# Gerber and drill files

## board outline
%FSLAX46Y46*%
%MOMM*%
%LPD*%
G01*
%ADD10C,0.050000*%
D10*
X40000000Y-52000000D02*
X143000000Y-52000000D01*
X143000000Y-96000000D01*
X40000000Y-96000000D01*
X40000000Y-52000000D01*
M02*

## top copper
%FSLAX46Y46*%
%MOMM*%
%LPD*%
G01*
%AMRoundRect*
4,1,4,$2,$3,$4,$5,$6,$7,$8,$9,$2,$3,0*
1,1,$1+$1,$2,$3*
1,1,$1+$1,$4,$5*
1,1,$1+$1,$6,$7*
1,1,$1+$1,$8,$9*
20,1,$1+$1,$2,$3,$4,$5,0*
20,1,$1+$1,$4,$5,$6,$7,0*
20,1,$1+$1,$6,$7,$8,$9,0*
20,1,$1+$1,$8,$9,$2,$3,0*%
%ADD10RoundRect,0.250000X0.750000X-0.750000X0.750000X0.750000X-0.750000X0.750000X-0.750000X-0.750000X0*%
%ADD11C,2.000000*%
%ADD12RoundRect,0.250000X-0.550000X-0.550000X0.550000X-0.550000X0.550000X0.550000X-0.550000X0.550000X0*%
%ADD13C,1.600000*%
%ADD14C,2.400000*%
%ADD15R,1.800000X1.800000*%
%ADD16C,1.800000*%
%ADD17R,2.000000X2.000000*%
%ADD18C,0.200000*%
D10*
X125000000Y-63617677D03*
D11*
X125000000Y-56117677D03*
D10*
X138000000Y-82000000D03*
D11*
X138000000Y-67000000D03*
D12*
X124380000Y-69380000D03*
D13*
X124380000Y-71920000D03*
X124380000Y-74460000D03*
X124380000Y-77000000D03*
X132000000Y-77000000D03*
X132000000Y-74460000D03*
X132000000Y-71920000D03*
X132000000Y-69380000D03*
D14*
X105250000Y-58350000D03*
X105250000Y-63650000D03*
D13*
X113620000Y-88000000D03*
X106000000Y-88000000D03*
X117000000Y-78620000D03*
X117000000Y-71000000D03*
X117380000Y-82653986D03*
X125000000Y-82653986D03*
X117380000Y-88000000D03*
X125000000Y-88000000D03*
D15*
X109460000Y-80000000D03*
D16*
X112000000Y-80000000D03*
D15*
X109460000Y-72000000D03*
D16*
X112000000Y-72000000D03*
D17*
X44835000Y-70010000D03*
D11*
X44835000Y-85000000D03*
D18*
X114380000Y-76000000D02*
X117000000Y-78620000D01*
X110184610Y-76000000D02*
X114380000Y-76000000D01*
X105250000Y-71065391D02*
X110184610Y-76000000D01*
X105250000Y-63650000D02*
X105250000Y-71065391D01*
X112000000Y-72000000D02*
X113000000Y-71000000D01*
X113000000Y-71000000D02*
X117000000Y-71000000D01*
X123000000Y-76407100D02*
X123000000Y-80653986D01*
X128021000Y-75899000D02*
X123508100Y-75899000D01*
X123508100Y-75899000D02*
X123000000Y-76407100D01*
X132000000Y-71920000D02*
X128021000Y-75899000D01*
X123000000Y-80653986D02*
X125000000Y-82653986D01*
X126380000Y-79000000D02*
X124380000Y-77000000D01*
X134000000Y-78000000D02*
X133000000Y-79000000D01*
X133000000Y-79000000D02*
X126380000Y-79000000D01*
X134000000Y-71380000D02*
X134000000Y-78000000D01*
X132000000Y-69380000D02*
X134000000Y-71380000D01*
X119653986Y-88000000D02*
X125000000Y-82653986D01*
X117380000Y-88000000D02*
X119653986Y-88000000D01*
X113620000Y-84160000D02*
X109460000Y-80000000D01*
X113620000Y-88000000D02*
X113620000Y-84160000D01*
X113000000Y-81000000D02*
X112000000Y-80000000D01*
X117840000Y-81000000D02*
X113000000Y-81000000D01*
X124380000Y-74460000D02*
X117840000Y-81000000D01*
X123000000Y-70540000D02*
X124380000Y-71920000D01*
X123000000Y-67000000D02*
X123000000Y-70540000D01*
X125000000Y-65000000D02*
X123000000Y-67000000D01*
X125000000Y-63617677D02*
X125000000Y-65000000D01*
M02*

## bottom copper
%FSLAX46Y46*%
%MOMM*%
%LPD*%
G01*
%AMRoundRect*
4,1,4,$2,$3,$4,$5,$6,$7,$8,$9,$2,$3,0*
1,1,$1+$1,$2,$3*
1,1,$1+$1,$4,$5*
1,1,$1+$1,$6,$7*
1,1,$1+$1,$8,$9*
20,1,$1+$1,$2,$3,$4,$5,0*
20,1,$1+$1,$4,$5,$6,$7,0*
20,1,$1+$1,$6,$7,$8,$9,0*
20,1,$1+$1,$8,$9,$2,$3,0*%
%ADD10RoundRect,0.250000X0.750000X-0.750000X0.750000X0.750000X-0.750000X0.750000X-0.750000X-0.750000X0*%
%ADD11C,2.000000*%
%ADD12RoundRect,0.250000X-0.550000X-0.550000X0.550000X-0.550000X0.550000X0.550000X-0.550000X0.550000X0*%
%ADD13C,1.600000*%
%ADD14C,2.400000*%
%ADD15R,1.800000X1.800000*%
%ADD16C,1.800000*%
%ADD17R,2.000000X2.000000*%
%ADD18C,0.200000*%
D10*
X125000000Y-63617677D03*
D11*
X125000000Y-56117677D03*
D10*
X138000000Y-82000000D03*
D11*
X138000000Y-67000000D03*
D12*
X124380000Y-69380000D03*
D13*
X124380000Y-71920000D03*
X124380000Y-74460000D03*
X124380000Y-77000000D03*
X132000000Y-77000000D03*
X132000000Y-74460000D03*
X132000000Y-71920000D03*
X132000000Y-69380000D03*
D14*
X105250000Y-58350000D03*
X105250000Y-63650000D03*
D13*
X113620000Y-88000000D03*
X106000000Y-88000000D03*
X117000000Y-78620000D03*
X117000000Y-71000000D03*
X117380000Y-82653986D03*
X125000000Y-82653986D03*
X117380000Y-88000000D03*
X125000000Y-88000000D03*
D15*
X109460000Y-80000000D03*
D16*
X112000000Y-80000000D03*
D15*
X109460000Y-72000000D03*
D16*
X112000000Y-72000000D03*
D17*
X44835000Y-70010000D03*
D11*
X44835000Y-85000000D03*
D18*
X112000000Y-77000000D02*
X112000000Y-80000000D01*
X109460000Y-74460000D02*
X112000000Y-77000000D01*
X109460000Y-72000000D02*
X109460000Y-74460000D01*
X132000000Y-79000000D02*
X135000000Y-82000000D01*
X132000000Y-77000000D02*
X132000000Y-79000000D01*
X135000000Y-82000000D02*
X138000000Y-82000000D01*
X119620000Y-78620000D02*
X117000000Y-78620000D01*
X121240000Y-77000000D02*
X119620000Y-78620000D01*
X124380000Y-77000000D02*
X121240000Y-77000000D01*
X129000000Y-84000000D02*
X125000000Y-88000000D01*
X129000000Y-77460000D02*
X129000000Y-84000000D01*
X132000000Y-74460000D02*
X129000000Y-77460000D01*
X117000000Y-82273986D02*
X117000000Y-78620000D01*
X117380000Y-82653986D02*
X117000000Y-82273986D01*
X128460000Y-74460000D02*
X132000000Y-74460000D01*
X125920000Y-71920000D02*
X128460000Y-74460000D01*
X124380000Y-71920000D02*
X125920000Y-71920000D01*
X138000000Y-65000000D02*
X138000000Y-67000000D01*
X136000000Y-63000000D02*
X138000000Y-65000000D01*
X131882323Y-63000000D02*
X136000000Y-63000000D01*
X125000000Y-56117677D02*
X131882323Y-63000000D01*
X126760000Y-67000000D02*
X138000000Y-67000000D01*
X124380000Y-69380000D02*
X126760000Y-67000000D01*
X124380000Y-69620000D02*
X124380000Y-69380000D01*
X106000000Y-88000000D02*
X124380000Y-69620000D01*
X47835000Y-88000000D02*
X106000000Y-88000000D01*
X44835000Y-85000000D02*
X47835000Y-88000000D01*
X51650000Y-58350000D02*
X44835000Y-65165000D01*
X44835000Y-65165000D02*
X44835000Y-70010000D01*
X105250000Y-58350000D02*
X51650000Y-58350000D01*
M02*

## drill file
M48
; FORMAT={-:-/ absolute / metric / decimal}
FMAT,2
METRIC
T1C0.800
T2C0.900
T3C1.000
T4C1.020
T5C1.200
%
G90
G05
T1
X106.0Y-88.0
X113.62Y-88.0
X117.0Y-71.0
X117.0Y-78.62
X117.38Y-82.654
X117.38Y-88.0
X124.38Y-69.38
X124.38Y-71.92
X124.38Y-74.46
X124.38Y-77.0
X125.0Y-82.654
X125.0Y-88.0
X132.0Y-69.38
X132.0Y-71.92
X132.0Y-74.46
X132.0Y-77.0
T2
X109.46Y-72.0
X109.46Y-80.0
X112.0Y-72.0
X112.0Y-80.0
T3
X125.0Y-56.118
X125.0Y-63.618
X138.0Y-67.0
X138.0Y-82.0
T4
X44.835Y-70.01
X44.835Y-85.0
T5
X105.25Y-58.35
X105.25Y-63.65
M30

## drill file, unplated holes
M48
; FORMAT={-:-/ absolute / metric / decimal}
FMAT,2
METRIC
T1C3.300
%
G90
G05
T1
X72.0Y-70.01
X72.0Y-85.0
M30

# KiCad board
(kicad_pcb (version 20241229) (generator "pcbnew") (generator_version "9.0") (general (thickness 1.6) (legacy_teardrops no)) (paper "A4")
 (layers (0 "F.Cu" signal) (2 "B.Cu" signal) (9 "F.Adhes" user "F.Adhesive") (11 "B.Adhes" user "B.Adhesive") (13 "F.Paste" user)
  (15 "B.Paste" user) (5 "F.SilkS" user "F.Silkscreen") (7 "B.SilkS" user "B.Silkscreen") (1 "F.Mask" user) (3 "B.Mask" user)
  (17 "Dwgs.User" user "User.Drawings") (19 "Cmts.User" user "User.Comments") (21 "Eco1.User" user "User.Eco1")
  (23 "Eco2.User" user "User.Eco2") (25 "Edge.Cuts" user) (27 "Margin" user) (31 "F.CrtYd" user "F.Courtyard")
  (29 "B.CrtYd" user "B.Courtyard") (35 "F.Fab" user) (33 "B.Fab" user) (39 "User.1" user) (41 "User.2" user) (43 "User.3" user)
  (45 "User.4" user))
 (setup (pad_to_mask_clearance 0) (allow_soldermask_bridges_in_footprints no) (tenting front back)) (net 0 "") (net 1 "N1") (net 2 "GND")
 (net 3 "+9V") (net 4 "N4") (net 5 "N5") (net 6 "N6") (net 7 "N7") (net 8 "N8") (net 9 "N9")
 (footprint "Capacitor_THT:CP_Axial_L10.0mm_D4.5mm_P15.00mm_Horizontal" (layer "F.Cu") (at 138 82 90)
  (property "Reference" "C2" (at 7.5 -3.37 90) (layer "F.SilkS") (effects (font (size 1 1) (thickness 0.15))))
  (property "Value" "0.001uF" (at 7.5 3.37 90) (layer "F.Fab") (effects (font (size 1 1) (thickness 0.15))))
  (pad "1" thru_hole roundrect (at 0 0 90) (size 2 2) (drill 1) (layers "*.Cu" "*.Mask") (remove_unused_layers no) (roundrect_rratio 0.125)
   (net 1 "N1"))
  (pad "2" thru_hole circle (at 15 0 90) (size 2 2) (drill 1) (layers "*.Cu" "*.Mask") (remove_unused_layers no) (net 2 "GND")))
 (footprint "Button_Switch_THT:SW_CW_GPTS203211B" (layer "F.Cu") (at 105.25 58.35)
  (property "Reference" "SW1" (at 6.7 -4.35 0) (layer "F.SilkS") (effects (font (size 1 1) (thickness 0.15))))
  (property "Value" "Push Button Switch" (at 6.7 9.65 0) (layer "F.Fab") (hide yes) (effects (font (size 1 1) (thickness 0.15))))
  (pad "1" thru_hole circle (at 0 0) (size 2.4 2.4) (drill 1.2) (layers "*.Cu" "*.Mask") (remove_unused_layers no) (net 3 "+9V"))
  (pad "2" thru_hole circle (at 0 5.3) (size 2.4 2.4) (drill 1.2) (layers "*.Cu" "*.Mask") (remove_unused_layers no) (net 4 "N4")))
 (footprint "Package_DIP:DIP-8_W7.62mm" (layer "F.Cu") (at 124.38 69.38)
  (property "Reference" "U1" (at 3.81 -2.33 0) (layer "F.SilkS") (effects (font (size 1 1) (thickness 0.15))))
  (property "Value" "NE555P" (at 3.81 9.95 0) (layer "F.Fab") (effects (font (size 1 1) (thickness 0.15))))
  (pad "1" thru_hole roundrect (at 0 0) (size 1.6 1.6) (drill 0.8) (layers "*.Cu" "*.Mask") (remove_unused_layers no)
   (roundrect_rratio 0.15625) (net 2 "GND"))
  (pad "2" thru_hole circle (at 0 2.54) (size 1.6 1.6) (drill 0.8) (layers "*.Cu" "*.Mask") (remove_unused_layers no) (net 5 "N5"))
  (pad "3" thru_hole circle (at 0 5.08) (size 1.6 1.6) (drill 0.8) (layers "*.Cu" "*.Mask") (remove_unused_layers no) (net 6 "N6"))
  (pad "4" thru_hole circle (at 0 7.62) (size 1.6 1.6) (drill 0.8) (layers "*.Cu" "*.Mask") (remove_unused_layers no) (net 4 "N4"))
  (pad "5" thru_hole circle (at 7.62 7.62) (size 1.6 1.6) (drill 0.8) (layers "*.Cu" "*.Mask") (remove_unused_layers no) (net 1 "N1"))
  (pad "6" thru_hole circle (at 7.62 5.08) (size 1.6 1.6) (drill 0.8) (layers "*.Cu" "*.Mask") (remove_unused_layers no) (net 5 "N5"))
  (pad "7" thru_hole circle (at 7.62 2.54) (size 1.6 1.6) (drill 0.8) (layers "*.Cu" "*.Mask") (remove_unused_layers no) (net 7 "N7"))
  (pad "8" thru_hole circle (at 7.62 0) (size 1.6 1.6) (drill 0.8) (layers "*.Cu" "*.Mask") (remove_unused_layers no) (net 4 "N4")))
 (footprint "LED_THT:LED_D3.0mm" (layer "F.Cu") (at 109.46 80)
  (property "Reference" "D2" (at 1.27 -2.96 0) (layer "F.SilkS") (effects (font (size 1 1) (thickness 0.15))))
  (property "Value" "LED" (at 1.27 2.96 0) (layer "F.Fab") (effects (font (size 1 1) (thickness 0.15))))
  (pad "1" thru_hole rect (at 0 0) (size 1.8 1.8) (drill 0.9) (layers "*.Cu" "*.Mask") (remove_unused_layers no) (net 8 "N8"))
  (pad "2" thru_hole circle (at 2.54 0) (size 1.8 1.8) (drill 0.9) (layers "*.Cu" "*.Mask") (remove_unused_layers no) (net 6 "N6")))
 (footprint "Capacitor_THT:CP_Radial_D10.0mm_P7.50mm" (layer "F.Cu") (at 125 63.617677 90)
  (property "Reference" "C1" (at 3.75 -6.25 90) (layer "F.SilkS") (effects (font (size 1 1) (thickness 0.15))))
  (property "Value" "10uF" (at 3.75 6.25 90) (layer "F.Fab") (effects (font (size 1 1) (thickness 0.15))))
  (pad "1" thru_hole roundrect (at 0 0 90) (size 2 2) (drill 1) (layers "*.Cu" "*.Mask") (remove_unused_layers no) (roundrect_rratio 0.125)
   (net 5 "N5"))
  (pad "2" thru_hole circle (at 7.5 0 90) (size 2 2) (drill 1) (layers "*.Cu" "*.Mask") (remove_unused_layers no) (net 2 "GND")))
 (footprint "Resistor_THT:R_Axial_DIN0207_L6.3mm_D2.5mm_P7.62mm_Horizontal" (layer "F.Cu") (at 117.38 88)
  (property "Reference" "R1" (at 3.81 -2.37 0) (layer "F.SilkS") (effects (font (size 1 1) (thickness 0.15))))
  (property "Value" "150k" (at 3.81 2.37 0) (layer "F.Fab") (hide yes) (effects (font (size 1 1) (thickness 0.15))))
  (pad "1" thru_hole circle (at 0 0) (size 1.6 1.6) (drill 0.8) (layers "*.Cu" "*.Mask") (remove_unused_layers no) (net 7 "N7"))
  (pad "2" thru_hole circle (at 7.62 0) (size 1.6 1.6) (drill 0.8) (layers "*.Cu" "*.Mask") (remove_unused_layers no) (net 5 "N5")))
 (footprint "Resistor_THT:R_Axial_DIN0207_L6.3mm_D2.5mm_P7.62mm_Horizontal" (layer "F.Cu") (at 113.62 88 180)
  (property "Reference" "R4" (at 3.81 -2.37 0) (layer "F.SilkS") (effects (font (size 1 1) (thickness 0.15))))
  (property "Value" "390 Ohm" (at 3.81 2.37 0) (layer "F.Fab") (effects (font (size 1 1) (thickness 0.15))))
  (pad "1" thru_hole circle (at 0 0 180) (size 1.6 1.6) (drill 0.8) (layers "*.Cu" "*.Mask") (remove_unused_layers no) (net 8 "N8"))
  (pad "2" thru_hole circle (at 7.62 0 180) (size 1.6 1.6) (drill 0.8) (layers "*.Cu" "*.Mask") (remove_unused_layers no) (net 2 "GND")))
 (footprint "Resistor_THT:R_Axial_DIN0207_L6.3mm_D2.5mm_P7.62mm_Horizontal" (layer "F.Cu") (at 117.38 82.653986)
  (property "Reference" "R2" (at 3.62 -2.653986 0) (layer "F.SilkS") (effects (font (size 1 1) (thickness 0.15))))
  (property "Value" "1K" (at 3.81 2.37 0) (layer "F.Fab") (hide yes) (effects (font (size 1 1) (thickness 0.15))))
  (pad "1" thru_hole circle (at 0 0) (size 1.6 1.6) (drill 0.8) (layers "*.Cu" "*.Mask") (remove_unused_layers no) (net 4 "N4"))
  (pad "2" thru_hole circle (at 7.62 0) (size 1.6 1.6) (drill 0.8) (layers "*.Cu" "*.Mask") (remove_unused_layers no) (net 7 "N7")))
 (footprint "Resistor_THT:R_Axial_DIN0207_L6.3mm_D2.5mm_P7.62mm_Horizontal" (layer "F.Cu") (at 117 78.62 90)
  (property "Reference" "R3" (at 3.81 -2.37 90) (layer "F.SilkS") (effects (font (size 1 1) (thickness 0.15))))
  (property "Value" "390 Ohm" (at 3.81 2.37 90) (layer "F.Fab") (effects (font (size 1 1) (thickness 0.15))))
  (pad "1" thru_hole circle (at 0 0 90) (size 1.6 1.6) (drill 0.8) (layers "*.Cu" "*.Mask") (remove_unused_layers no) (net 4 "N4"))
  (pad "2" thru_hole circle (at 7.62 0 90) (size 1.6 1.6) (drill 0.8) (layers "*.Cu" "*.Mask") (remove_unused_layers no) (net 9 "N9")))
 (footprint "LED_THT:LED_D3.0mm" (layer "F.Cu") (at 109.46 72)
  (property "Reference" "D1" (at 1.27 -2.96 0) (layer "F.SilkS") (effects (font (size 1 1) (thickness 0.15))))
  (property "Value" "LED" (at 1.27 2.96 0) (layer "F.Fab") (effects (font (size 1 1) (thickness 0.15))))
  (pad "1" thru_hole rect (at 0 0) (size 1.8 1.8) (drill 0.9) (layers "*.Cu" "*.Mask") (remove_unused_layers no) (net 6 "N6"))
  (pad "2" thru_hole circle (at 2.54 0) (size 1.8 1.8) (drill 0.9) (layers "*.Cu" "*.Mask") (remove_unused_layers no) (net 9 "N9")))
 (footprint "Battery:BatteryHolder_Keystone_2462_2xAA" (layer "F.Cu") (at 44.835 70.01)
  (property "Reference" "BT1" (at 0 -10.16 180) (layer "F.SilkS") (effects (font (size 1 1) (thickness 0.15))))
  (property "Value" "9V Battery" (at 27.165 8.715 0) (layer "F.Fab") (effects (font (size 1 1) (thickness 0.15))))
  (pad "" np_thru_hole circle (at 27.165 0) (size 3.3 3.3) (drill 3.3) (layers "*.Cu" "*.Mask"))
  (pad "" np_thru_hole circle (at 27.165 14.99) (size 3.3 3.3) (drill 3.3) (layers "*.Cu" "*.Mask"))
  (pad "1" thru_hole rect (at 0 0) (size 2 2) (drill 1.02) (layers "*.Cu" "*.Mask") (remove_unused_layers no) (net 3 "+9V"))
  (pad "2" thru_hole circle (at 0 14.99) (size 2 2) (drill 1.02) (layers "*.Cu" "*.Mask") (remove_unused_layers no) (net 2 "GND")))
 (gr_rect (start 40 52) (end 143 96) (stroke (width 0.05) (type default)) (fill no) (layer "Edge.Cuts"))
 (segment (start 44.835 85) (end 47.835 88) (width 0.2) (layer "B.Cu") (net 2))
 (segment (start 131.882323 63) (end 136 63) (width 0.2) (layer "B.Cu") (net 2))
 (segment (start 47.835 88) (end 106 88) (width 0.2) (layer "B.Cu") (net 2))
 (segment (start 106 88) (end 124.38 69.62) (width 0.2) (layer "B.Cu") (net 2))
 (segment (start 126.76 67) (end 138 67) (width 0.2) (layer "B.Cu") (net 2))
 (segment (start 138 65) (end 138 67) (width 0.2) (layer "B.Cu") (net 2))
 (segment (start 125 56.117677) (end 131.882323 63) (width 0.2) (layer "B.Cu") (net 2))
 (segment (start 136 63) (end 138 65) (width 0.2) (layer "B.Cu") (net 2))
 (segment (start 124.38 69.38) (end 126.76 67) (width 0.2) (layer "B.Cu") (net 2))
 (segment (start 124.38 69.62) (end 124.38 69.38) (width 0.2) (layer "B.Cu") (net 2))
 (segment (start 44.835 65.165) (end 44.835 70.01) (width 0.2) (layer "B.Cu") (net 3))
 (segment (start 51.65 58.35) (end 44.835 65.165) (width 0.2) (layer "B.Cu") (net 3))
 (segment (start 105.25 58.35) (end 51.65 58.35) (width 0.2) (layer "B.Cu") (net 3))
 (segment (start 123 70.54) (end 124.38 71.92) (width 0.2) (layer "F.Cu") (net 5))
 (segment (start 125 63.617677) (end 125 65) (width 0.2) (layer "F.Cu") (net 5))
 (segment (start 125 65) (end 123 67) (width 0.2) (layer "F.Cu") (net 5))
 (segment (start 123 67) (end 123 70.54) (width 0.2) (layer "F.Cu") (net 5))
 (segment (start 128.46 74.46) (end 132 74.46) (width 0.2) (layer "B.Cu") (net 5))
 (segment (start 124.38 71.92) (end 125.92 71.92) (width 0.2) (layer "B.Cu") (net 5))
 (segment (start 132 74.46) (end 129 77.46) (width 0.2) (layer "B.Cu") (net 5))
 (segment (start 129 77.46) (end 129 84) (width 0.2) (layer "B.Cu") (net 5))
 (segment (start 129 84) (end 125 88) (width 0.2) (layer "B.Cu") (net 5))
 (segment (start 125.92 71.92) (end 128.46 74.46) (width 0.2) (layer "B.Cu") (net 5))
 (segment (start 132 77) (end 132 79) (width 0.2) (layer "B.Cu") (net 1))
 (segment (start 132 79) (end 135 82) (width 0.2) (layer "B.Cu") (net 1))
 (segment (start 135 82) (end 138 82) (width 0.2) (layer "B.Cu") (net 1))
 (segment (start 117.84 81) (end 113 81) (width 0.2) (layer "F.Cu") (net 6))
 (segment (start 124.38 74.46) (end 117.84 81) (width 0.2) (layer "F.Cu") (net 6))
 (segment (start 113 81) (end 112 80) (width 0.2) (layer "F.Cu") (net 6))
 (segment (start 109.46 72) (end 109.46 74.46) (width 0.2) (layer "B.Cu") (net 6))
 (segment (start 109.46 74.46) (end 112 77) (width 0.2) (layer "B.Cu") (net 6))
 (segment (start 112 77) (end 112 80) (width 0.2) (layer "B.Cu") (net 6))
 (segment (start 112 72) (end 113 71) (width 0.2) (layer "F.Cu") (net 9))
 (segment (start 113 71) (end 117 71) (width 0.2) (layer "F.Cu") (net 9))
 (segment (start 113.62 84.16) (end 109.46 80) (width 0.2) (layer "F.Cu") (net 8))
 (segment (start 113.62 88) (end 113.62 84.16) (width 0.2) (layer "F.Cu") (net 8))
 (segment (start 123 76.4071) (end 123 80.653986) (width 0.2) (layer "F.Cu") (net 7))
 (segment (start 123 80.653986) (end 125 82.653986) (width 0.2) (layer "F.Cu") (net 7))
 (segment (start 123.5081 75.899) (end 123 76.4071) (width 0.2) (layer "F.Cu") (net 7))
 (segment (start 119.653986 88) (end 125 82.653986) (width 0.2) (layer "F.Cu") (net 7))
 (segment (start 128.021 75.899) (end 123.5081 75.899) (width 0.2) (layer "F.Cu") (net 7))
 (segment (start 117.38 88) (end 119.653986 88) (width 0.2) (layer "F.Cu") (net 7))
 (segment (start 132 71.92) (end 128.021 75.899) (width 0.2) (layer "F.Cu") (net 7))
 (segment (start 126.38 79) (end 124.38 77) (width 0.2) (layer "F.Cu") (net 4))
 (segment (start 110.18461 76) (end 114.38 76) (width 0.2) (layer "F.Cu") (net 4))
 (segment (start 105.25 71.065391) (end 110.18461 76) (width 0.2) (layer "F.Cu") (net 4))
 (segment (start 114.38 76) (end 117 78.62) (width 0.2) (layer "F.Cu") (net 4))
 (segment (start 134 71.38) (end 134 78) (width 0.2) (layer "F.Cu") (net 4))
 (segment (start 134 78) (end 133 79) (width 0.2) (layer "F.Cu") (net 4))
 (segment (start 133 79) (end 126.38 79) (width 0.2) (layer "F.Cu") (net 4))
 (segment (start 132 69.38) (end 134 71.38) (width 0.2) (layer "F.Cu") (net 4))
 (segment (start 105.25 63.65) (end 105.25 71.065391) (width 0.2) (layer "F.Cu") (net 4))
 (segment (start 117 82.273986) (end 117 78.62) (width 0.2) (layer "B.Cu") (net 4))
 (segment (start 117.38 82.653986) (end 117 82.273986) (width 0.2) (layer "B.Cu") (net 4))
 (segment (start 124.38 77) (end 121.24 77) (width 0.2) (layer "B.Cu") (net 4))
 (segment (start 121.24 77) (end 119.62 78.62) (width 0.2) (layer "B.Cu") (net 4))
 (segment (start 119.62 78.62) (end 117 78.62) (width 0.2) (layer "B.Cu") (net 4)))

